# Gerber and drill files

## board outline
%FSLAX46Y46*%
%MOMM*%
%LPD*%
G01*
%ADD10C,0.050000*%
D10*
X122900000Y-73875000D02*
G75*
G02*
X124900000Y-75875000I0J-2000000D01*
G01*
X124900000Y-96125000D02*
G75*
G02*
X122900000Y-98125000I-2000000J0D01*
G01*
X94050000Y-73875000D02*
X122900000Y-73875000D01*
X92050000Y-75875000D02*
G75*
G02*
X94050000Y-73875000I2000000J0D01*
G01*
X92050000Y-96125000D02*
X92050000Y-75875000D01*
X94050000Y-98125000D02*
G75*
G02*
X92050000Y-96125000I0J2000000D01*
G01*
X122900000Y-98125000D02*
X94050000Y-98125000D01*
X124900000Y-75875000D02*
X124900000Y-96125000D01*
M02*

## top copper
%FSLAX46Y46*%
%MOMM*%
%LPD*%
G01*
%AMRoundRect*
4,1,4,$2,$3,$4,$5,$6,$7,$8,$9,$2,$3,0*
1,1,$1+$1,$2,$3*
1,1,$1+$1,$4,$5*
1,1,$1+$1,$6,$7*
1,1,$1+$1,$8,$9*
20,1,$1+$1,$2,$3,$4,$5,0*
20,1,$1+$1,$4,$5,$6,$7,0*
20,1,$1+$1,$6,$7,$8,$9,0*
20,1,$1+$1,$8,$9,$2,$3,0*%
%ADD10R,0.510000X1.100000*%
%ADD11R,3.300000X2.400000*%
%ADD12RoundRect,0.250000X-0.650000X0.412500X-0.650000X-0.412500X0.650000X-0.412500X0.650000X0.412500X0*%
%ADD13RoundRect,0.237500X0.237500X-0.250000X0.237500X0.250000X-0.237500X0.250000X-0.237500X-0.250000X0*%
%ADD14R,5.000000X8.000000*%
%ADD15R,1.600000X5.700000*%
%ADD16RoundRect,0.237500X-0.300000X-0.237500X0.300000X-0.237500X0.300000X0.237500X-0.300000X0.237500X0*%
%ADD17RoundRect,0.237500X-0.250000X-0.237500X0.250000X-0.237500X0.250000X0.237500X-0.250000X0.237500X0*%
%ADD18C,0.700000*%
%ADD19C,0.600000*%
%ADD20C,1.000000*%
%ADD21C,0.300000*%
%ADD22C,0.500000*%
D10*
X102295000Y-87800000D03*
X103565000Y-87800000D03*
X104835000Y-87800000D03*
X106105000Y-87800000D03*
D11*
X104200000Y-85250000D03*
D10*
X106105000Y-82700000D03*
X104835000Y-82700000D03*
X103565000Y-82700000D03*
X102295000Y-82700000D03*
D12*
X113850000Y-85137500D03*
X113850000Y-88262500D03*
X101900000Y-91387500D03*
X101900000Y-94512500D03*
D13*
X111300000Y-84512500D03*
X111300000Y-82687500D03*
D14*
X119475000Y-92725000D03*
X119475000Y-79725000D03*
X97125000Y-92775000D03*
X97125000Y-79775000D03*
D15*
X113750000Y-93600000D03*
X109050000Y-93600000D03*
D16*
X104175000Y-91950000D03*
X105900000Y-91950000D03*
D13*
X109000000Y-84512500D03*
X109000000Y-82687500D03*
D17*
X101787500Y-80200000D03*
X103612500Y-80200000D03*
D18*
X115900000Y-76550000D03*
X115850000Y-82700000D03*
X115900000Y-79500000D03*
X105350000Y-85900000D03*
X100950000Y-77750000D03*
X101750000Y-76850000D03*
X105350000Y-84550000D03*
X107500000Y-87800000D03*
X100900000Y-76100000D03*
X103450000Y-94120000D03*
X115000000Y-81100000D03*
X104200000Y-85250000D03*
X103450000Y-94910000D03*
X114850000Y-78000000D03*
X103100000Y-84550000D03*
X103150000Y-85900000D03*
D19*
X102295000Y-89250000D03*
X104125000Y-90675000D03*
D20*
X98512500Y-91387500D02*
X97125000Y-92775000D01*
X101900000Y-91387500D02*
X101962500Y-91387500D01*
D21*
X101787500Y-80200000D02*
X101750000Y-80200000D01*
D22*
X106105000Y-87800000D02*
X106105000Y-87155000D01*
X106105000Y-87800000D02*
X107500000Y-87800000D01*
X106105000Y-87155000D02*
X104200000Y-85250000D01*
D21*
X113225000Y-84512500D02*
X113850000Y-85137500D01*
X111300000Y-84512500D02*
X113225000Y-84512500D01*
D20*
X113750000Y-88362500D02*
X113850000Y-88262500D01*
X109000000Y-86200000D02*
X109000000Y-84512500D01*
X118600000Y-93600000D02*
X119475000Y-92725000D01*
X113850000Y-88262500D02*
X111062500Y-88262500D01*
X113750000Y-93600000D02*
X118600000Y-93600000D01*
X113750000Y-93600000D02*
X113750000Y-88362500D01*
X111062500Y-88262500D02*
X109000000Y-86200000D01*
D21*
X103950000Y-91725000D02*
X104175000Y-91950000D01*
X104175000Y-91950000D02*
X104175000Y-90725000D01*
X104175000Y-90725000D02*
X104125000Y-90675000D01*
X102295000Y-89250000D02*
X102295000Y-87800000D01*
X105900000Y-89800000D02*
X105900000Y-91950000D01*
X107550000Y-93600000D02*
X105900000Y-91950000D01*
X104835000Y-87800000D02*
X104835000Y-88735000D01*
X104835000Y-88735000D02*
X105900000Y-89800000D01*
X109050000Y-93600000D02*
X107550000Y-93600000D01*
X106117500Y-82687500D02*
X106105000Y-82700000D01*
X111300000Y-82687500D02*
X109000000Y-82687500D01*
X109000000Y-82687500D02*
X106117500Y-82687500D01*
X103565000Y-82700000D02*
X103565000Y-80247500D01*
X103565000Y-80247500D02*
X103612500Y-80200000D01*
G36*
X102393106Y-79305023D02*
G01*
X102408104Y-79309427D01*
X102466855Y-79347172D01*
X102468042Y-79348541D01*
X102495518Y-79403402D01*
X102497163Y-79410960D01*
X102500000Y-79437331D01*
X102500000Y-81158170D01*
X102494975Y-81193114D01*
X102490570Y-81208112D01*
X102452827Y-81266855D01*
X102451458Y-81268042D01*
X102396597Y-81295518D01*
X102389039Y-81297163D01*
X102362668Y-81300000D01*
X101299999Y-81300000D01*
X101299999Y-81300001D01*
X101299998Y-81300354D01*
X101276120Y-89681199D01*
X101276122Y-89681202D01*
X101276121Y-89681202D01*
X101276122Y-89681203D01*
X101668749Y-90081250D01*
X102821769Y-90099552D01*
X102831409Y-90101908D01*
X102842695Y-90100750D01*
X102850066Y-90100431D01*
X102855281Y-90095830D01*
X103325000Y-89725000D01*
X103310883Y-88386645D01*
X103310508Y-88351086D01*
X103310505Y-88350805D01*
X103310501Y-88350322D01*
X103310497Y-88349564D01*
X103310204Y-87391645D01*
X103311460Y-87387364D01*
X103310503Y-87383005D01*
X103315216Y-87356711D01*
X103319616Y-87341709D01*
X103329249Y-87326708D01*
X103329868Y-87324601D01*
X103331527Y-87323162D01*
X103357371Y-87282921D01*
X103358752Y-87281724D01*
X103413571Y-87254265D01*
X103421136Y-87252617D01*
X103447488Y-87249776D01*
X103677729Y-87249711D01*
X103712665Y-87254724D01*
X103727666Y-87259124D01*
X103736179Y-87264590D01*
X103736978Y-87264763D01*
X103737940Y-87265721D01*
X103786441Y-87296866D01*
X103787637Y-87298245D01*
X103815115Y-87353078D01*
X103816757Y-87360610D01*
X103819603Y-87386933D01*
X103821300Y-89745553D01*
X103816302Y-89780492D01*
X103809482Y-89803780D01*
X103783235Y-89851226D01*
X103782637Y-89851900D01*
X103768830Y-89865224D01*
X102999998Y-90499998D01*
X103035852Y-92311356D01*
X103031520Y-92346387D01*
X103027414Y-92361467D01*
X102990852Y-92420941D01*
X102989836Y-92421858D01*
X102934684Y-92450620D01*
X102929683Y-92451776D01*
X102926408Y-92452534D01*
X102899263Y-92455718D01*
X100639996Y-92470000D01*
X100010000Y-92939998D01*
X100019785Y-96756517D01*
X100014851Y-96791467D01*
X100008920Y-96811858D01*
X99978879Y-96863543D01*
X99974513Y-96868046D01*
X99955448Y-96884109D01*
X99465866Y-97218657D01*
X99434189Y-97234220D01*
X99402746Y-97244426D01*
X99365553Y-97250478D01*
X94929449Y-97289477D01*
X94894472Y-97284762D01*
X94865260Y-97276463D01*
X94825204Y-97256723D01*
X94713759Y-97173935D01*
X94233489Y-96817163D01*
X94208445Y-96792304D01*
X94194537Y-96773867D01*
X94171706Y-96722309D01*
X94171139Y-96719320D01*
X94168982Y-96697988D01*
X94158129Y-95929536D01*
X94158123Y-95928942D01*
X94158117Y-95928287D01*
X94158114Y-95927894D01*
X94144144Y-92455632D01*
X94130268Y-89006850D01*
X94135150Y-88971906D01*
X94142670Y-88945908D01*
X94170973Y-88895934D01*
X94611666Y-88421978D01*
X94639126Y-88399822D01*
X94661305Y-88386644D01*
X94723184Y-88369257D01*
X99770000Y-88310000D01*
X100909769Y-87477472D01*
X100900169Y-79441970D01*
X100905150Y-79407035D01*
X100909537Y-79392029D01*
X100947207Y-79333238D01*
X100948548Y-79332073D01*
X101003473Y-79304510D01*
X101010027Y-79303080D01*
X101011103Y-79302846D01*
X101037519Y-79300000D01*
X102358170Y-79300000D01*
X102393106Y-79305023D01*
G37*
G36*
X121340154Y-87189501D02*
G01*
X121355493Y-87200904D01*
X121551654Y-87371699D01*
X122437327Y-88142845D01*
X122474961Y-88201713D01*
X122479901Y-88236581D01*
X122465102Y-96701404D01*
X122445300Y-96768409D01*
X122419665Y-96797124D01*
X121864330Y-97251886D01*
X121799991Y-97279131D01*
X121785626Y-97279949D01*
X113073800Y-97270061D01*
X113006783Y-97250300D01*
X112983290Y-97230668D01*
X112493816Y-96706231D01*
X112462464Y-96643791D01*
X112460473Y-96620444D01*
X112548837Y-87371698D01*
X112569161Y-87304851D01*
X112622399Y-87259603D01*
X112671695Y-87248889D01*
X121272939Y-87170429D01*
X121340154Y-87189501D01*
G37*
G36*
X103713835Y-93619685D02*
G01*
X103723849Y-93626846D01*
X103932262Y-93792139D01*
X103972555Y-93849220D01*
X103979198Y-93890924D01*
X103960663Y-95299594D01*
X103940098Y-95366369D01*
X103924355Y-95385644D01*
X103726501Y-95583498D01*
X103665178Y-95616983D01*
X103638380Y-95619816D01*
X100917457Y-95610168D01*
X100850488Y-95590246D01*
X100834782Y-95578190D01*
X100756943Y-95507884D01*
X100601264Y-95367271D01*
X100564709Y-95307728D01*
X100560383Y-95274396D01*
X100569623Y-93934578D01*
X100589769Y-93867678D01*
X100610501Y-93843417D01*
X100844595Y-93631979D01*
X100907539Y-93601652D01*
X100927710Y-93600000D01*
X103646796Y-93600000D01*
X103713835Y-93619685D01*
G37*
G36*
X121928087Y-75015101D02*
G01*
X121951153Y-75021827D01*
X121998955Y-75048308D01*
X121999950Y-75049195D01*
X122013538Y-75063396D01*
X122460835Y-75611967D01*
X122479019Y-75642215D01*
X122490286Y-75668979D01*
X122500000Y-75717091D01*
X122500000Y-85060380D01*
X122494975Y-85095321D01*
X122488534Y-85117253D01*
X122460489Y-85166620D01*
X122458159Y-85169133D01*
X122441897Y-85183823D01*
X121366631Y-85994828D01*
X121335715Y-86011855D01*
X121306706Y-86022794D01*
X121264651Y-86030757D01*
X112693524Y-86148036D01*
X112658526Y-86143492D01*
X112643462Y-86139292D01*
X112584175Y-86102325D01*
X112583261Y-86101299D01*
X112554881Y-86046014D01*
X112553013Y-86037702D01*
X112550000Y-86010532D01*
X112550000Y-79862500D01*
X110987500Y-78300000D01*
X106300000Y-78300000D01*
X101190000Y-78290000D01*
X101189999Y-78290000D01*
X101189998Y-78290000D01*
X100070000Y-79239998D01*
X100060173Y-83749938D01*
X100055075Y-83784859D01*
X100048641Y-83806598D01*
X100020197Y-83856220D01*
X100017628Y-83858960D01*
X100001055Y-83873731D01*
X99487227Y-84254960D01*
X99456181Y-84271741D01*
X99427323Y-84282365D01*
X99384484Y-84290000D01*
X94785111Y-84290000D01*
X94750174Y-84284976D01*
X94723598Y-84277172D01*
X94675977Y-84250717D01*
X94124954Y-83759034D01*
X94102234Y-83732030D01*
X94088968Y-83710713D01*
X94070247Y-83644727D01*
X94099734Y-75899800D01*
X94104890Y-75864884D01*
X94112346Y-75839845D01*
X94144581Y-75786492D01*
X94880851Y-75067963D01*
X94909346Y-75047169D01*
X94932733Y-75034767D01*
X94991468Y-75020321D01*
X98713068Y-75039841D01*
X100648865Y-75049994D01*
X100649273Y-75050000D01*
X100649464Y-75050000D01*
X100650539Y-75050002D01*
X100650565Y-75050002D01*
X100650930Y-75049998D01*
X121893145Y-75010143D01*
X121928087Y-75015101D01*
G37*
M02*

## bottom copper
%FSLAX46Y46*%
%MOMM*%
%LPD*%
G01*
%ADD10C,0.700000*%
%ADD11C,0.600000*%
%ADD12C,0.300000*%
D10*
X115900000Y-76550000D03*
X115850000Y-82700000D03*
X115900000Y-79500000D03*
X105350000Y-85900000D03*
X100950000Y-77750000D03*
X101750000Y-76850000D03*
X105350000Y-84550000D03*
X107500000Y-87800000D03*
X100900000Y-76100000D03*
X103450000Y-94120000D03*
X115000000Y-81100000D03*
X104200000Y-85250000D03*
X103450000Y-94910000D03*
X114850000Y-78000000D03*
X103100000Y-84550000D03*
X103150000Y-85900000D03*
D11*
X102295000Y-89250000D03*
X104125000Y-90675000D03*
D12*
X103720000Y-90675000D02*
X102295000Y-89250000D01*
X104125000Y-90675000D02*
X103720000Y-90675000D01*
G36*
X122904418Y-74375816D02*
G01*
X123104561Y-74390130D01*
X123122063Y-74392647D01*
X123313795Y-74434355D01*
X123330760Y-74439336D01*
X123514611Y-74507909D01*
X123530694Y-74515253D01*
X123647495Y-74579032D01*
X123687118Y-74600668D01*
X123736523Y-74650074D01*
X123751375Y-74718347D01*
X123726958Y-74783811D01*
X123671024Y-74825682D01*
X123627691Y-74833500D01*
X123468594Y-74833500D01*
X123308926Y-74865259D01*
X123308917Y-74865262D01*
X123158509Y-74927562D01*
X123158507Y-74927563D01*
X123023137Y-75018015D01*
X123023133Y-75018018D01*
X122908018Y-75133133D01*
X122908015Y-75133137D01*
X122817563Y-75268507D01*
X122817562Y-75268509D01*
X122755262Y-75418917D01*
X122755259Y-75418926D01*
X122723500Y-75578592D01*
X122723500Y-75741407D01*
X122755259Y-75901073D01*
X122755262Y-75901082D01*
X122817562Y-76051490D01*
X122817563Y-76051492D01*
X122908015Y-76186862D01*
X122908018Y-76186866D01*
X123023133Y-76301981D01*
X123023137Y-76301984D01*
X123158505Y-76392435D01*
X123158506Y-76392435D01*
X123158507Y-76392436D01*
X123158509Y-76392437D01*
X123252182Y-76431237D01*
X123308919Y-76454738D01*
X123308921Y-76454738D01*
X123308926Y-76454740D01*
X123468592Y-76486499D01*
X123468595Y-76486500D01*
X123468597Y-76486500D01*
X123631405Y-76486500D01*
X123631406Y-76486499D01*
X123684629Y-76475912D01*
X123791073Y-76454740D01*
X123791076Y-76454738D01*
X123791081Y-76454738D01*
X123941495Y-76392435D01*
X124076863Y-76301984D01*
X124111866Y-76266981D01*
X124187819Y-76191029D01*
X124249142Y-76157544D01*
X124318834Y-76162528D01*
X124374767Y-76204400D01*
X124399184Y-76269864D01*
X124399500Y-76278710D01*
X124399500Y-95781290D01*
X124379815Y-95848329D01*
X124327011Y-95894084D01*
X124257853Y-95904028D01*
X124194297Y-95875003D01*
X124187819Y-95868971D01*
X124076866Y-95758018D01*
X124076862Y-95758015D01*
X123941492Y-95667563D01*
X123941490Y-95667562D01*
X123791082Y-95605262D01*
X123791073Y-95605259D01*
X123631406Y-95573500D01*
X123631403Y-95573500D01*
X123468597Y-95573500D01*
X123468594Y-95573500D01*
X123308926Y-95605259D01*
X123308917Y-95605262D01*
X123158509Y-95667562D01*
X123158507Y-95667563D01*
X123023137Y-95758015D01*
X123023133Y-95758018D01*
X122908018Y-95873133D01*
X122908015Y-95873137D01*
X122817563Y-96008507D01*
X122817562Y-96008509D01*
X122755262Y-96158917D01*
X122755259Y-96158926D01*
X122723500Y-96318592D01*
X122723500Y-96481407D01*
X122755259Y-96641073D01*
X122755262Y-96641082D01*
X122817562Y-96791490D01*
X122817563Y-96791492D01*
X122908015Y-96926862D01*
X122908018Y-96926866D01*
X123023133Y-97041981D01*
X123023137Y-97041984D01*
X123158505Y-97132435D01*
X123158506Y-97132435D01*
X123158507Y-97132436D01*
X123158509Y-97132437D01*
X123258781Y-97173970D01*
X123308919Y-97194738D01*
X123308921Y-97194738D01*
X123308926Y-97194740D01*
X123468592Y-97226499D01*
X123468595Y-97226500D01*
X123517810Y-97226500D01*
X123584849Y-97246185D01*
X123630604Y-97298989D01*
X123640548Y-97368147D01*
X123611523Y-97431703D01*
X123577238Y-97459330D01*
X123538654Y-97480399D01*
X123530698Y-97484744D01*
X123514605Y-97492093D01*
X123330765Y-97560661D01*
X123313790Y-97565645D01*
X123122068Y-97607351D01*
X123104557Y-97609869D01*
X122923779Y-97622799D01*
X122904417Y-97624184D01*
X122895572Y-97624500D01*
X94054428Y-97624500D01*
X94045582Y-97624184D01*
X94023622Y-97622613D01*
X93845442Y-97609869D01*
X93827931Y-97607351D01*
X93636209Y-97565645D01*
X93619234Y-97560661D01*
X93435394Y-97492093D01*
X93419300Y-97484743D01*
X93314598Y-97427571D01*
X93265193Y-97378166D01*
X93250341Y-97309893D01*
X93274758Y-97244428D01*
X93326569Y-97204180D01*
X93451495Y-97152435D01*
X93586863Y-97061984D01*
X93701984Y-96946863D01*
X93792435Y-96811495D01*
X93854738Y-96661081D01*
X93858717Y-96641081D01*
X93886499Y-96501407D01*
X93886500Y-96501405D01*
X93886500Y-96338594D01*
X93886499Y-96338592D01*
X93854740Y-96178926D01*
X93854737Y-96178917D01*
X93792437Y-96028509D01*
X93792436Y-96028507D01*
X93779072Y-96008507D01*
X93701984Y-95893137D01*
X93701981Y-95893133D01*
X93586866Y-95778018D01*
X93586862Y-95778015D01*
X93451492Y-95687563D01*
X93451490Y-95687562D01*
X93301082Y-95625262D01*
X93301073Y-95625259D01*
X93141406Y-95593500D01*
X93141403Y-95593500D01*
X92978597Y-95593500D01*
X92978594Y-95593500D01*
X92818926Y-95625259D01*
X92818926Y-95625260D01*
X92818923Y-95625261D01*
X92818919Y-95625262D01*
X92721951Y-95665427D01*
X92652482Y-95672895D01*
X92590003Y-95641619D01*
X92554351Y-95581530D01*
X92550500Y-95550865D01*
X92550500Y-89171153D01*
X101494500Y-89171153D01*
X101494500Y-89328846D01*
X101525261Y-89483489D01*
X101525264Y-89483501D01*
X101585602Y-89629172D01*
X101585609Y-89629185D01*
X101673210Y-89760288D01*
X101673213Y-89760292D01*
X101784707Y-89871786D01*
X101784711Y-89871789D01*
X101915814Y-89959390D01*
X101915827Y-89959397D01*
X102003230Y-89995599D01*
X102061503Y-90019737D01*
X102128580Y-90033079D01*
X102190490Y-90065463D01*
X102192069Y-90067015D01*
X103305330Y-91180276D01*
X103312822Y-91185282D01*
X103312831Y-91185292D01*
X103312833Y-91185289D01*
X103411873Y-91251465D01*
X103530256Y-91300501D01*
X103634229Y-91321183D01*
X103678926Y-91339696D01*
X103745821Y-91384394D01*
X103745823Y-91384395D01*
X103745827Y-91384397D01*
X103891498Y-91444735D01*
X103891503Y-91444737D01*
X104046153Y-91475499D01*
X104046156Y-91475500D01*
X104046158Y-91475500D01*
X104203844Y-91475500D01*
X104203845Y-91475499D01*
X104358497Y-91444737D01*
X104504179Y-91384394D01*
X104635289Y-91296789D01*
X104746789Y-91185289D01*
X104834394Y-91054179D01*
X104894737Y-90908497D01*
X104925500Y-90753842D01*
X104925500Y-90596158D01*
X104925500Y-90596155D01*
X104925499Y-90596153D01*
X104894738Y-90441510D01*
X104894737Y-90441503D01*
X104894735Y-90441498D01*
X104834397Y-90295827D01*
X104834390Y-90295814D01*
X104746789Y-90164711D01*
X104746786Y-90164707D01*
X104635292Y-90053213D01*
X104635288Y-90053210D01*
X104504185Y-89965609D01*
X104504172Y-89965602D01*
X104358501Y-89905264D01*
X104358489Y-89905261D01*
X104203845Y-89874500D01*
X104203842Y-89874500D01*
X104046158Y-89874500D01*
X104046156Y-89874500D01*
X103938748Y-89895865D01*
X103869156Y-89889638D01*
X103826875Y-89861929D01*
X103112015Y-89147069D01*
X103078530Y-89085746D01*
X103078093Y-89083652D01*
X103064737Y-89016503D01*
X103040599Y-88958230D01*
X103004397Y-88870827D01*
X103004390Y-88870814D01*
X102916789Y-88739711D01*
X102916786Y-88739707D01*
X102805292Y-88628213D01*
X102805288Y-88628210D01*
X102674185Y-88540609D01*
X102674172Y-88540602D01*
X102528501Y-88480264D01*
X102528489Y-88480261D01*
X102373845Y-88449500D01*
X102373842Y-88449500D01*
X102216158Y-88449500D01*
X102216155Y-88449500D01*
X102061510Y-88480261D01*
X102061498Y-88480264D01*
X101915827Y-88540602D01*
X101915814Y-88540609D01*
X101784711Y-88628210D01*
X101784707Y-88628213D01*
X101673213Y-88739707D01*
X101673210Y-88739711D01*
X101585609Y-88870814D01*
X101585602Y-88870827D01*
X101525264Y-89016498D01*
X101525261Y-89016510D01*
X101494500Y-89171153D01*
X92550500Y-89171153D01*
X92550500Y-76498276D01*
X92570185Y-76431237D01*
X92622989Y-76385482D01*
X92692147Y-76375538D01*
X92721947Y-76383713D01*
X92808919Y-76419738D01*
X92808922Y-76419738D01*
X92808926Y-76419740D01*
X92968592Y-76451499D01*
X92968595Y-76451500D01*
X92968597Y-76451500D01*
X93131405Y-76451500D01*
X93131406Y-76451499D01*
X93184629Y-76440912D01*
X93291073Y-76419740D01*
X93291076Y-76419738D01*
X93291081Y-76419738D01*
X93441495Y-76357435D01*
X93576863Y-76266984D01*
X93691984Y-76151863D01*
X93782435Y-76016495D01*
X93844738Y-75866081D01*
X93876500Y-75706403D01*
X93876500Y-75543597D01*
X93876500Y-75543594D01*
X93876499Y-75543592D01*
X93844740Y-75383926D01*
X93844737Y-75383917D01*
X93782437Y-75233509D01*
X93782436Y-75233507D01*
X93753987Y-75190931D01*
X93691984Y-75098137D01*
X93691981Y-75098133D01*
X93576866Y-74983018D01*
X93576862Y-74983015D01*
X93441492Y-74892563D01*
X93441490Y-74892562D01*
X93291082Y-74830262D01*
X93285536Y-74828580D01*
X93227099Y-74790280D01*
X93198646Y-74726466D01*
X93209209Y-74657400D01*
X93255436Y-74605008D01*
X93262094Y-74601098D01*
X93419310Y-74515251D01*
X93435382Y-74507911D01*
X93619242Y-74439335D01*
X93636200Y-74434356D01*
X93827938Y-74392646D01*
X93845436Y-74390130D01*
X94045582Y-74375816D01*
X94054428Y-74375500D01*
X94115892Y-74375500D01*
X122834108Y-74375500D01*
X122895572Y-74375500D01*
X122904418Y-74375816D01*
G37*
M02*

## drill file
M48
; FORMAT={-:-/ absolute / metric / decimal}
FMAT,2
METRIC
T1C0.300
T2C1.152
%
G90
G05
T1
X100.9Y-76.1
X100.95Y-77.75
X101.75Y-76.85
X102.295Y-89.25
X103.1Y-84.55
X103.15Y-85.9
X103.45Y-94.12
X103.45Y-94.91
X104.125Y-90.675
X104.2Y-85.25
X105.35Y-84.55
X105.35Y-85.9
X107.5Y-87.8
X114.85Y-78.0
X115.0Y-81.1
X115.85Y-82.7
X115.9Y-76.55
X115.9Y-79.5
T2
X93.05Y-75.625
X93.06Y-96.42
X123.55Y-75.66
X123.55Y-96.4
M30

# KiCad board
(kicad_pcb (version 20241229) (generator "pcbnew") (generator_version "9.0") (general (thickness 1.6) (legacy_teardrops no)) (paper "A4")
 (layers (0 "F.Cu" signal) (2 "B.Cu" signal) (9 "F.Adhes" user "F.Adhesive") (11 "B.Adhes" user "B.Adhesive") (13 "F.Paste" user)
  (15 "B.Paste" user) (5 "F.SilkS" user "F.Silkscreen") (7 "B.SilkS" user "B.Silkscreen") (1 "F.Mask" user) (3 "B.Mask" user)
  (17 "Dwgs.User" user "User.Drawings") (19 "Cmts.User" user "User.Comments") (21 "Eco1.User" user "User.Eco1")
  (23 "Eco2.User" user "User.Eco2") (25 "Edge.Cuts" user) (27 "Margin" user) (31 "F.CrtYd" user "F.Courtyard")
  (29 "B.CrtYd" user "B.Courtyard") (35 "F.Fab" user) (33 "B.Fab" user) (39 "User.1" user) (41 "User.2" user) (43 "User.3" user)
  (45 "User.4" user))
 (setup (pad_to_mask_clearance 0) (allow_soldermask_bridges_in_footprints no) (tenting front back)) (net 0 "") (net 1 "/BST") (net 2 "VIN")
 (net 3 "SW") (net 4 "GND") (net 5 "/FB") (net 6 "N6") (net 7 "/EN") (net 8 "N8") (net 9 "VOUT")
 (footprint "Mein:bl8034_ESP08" (layer "F.Cu") (at 104.2 85.25 90)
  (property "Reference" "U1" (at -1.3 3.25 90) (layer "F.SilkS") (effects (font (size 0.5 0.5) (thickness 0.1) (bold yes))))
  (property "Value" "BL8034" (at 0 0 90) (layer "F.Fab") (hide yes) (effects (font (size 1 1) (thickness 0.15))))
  (pad "1" smd rect (at -2.55 -1.905) (size 0.51 1.1) (layers "F.Cu" "F.Mask" "F.Paste") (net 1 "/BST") (thermal_bridge_angle 45))
  (pad "2" smd rect (at -2.55 -0.635) (size 0.51 1.1) (layers "F.Cu" "F.Mask" "F.Paste") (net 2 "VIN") (thermal_bridge_angle 45))
  (pad "3" smd rect (at -2.55 0.635) (size 0.51 1.1) (layers "F.Cu" "F.Mask" "F.Paste") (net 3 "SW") (thermal_bridge_angle 45))
  (pad "4" smd rect (at -2.55 1.905) (size 0.51 1.1) (layers "F.Cu" "F.Mask" "F.Paste") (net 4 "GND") (thermal_bridge_angle 45))
  (pad "4" smd rect (at 0 0) (size 3.3 2.4) (layers "F.Cu" "F.Mask" "F.Paste") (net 4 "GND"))
  (pad "5" smd rect (at 2.55 1.905) (size 0.51 1.1) (layers "F.Cu" "F.Mask" "F.Paste") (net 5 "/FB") (thermal_bridge_angle 45))
  (pad "6" smd rect (at 2.55 0.635) (size 0.51 1.1) (layers "F.Cu" "F.Mask" "F.Paste") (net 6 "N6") (thermal_bridge_angle 45))
  (pad "7" smd rect (at 2.55 -0.635) (size 0.51 1.1) (layers "F.Cu" "F.Mask" "F.Paste") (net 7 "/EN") (thermal_bridge_angle 45))
  (pad "8" smd rect (at 2.55 -1.905) (size 0.51 1.1) (layers "F.Cu" "F.Mask" "F.Paste") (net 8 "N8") (thermal_bridge_angle 45)))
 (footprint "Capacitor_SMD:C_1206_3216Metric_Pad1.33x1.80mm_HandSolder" (layer "F.Cu") (at 113.85 86.7 -90)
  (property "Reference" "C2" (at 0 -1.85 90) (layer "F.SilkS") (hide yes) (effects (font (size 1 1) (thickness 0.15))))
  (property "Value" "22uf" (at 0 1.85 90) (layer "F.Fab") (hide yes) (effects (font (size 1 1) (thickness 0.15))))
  (pad "1" smd roundrect (at -1.5625 0 270) (size 1.325 1.8) (layers "F.Cu" "F.Mask" "F.Paste") (roundrect_rratio 0.188679) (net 4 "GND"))
  (pad "2" smd roundrect (at 1.5625 0 270) (size 1.325 1.8) (layers "F.Cu" "F.Mask" "F.Paste") (roundrect_rratio 0.188679) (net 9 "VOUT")))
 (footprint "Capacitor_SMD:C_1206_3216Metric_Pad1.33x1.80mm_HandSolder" (layer "F.Cu") (at 101.9 92.95 -90)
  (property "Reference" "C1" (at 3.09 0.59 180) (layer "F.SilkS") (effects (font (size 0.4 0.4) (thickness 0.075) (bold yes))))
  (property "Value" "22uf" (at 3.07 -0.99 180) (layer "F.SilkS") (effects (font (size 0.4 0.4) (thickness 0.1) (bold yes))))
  (pad "1" smd roundrect (at -1.5625 0 270) (size 1.325 1.8) (layers "F.Cu" "F.Mask" "F.Paste") (roundrect_rratio 0.188679) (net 2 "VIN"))
  (pad "2" smd roundrect (at 1.5625 0 270) (size 1.325 1.8) (layers "F.Cu" "F.Mask" "F.Paste") (roundrect_rratio 0.188679) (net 4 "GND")))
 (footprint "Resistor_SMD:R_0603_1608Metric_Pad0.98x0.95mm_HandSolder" (layer "F.Cu") (at 111.3 83.6 90)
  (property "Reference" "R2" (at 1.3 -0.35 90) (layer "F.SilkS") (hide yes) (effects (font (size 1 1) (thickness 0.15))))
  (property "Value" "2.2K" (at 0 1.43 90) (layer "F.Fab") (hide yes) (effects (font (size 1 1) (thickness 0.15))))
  (pad "1" smd roundrect (at -0.9125 0 90) (size 0.975 0.95) (layers "F.Cu" "F.Mask" "F.Paste") (roundrect_rratio 0.25) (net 4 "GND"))
  (pad "2" smd roundrect (at 0.9125 0 90) (size 0.975 0.95) (layers "F.Cu" "F.Mask" "F.Paste") (roundrect_rratio 0.25) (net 5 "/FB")))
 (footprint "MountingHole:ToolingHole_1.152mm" (layer "F.Cu") (at 123.55 75.66)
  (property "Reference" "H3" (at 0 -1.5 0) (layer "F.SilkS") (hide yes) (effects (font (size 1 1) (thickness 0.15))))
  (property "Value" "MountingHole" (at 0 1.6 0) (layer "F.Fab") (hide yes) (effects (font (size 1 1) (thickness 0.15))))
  (pad "" np_thru_hole circle (at 0 0) (size 1.152 1.152) (drill 1.152) (layers "*.Cu" "*.Mask") (solder_mask_margin 0.074))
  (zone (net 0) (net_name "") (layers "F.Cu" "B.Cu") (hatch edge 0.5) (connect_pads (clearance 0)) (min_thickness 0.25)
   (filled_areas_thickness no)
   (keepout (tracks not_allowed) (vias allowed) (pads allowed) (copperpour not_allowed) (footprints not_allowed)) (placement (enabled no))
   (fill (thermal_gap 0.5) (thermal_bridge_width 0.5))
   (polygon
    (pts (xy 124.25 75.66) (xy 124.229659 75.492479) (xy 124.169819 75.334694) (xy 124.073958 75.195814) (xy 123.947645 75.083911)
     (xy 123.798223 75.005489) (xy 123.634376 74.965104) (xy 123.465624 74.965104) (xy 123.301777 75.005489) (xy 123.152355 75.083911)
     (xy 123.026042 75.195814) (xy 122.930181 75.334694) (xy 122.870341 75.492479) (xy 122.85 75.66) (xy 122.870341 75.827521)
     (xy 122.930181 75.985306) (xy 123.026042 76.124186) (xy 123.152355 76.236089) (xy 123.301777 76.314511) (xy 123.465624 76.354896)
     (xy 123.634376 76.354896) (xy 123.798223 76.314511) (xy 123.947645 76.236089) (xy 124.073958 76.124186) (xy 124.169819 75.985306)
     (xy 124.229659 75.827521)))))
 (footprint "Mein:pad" (layer "F.Cu") (at 116.975 102.225 180)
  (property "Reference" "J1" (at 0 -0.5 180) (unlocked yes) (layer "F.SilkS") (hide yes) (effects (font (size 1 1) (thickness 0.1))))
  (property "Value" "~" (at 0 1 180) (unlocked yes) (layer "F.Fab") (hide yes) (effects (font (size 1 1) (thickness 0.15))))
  (pad "1" smd rect (at -2.5 9.5 270) (size 8 5) (layers "F.Cu" "F.Mask" "F.Paste") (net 9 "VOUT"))
  (pad "2" smd rect (at -2.5 22.5 270) (size 8 5) (layers "F.Cu" "F.Mask" "F.Paste") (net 4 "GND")))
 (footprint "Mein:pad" (layer "F.Cu") (at 94.625 102.275 180)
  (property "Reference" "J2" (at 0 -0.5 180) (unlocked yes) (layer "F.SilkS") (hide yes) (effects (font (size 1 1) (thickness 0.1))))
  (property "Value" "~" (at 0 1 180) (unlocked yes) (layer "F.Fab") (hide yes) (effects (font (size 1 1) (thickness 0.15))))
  (pad "1" smd rect (at -2.5 9.5 270) (size 8 5) (layers "F.Cu" "F.Mask" "F.Paste") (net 2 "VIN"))
  (pad "2" smd rect (at -2.5 22.5 270) (size 8 5) (layers "F.Cu" "F.Mask" "F.Paste") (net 4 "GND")))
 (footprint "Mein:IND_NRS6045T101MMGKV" (layer "F.Cu") (at 111.4 93.6 180)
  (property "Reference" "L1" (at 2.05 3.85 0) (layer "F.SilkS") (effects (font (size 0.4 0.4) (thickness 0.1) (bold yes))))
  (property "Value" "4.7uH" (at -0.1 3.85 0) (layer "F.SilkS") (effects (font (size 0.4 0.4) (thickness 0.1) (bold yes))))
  (pad "1" smd rect (at -2.35 0 180) (size 1.6 5.7) (layers "F.Cu" "F.Mask" "F.Paste") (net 9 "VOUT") (solder_mask_margin 0.102))
  (pad "2" smd rect (at 2.35 0 180) (size 1.6 5.7) (layers "F.Cu" "F.Mask" "F.Paste") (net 3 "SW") (solder_mask_margin 0.102)))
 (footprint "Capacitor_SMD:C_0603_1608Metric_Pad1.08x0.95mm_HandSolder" (layer "F.Cu") (at 105.0375 91.95)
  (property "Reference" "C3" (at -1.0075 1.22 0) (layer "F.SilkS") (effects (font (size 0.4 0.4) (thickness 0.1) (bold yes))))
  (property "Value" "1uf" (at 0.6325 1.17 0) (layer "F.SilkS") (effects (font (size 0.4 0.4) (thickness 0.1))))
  (pad "1" smd roundrect (at -0.8625 0) (size 1.075 0.95) (layers "F.Cu" "F.Mask" "F.Paste") (roundrect_rratio 0.25) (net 1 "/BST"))
  (pad "2" smd roundrect (at 0.8625 0) (size 1.075 0.95) (layers "F.Cu" "F.Mask" "F.Paste") (roundrect_rratio 0.25) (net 3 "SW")))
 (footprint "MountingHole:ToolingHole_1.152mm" (layer "F.Cu") (at 93.05 75.625)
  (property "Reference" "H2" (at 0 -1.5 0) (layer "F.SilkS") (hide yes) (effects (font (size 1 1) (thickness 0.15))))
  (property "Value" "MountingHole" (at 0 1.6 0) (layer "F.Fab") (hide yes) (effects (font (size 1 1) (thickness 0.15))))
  (pad "" np_thru_hole circle (at 0 0) (size 1.152 1.152) (drill 1.152) (layers "*.Cu" "*.Mask") (solder_mask_margin 0.074))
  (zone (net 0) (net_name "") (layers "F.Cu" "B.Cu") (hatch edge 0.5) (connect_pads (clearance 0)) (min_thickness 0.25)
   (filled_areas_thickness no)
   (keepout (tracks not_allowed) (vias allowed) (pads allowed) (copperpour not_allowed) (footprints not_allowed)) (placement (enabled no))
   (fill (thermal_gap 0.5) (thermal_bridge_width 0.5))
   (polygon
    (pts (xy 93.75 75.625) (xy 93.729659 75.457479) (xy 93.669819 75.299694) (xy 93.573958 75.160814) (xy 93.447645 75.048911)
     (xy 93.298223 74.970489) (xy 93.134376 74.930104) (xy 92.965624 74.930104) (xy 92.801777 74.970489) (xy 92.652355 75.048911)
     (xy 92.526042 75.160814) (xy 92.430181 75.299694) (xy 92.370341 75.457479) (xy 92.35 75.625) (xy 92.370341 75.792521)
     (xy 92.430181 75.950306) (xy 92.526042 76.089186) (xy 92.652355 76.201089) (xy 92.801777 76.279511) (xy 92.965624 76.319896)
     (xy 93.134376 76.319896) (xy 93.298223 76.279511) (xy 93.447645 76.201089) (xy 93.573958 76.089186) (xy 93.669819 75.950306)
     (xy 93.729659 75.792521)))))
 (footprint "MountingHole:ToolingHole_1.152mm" (layer "F.Cu") (at 93.06 96.42)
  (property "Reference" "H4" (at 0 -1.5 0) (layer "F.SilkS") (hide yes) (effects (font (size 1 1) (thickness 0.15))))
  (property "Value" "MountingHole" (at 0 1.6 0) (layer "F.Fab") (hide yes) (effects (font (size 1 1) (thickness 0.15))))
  (pad "" np_thru_hole circle (at 0 0) (size 1.152 1.152) (drill 1.152) (layers "*.Cu" "*.Mask") (solder_mask_margin 0.074))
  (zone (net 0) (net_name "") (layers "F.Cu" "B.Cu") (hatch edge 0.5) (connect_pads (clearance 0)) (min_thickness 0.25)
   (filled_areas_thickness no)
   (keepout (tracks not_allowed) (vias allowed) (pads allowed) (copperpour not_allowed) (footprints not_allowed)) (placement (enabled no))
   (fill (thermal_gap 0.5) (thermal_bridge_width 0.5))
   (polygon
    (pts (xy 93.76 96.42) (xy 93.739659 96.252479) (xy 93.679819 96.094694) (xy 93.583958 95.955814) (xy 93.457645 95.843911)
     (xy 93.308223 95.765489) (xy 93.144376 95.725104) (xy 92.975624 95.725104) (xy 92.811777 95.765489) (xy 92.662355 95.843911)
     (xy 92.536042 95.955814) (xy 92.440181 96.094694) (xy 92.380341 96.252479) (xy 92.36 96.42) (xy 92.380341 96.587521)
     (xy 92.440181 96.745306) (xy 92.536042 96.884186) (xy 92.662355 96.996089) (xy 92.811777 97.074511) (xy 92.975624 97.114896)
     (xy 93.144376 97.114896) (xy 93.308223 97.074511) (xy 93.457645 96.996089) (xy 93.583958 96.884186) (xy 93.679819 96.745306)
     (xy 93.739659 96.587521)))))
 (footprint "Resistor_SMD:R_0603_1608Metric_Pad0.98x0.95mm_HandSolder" (layer "F.Cu") (at 109 83.6 90)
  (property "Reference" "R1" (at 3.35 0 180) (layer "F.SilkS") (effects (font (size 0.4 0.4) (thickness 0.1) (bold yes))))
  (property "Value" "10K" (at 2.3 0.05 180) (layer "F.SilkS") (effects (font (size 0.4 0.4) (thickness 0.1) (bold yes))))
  (pad "1" smd roundrect (at -0.9125 0 90) (size 0.975 0.95) (layers "F.Cu" "F.Mask" "F.Paste") (roundrect_rratio 0.25) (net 9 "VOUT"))
  (pad "2" smd roundrect (at 0.9125 0 90) (size 0.975 0.95) (layers "F.Cu" "F.Mask" "F.Paste") (roundrect_rratio 0.25) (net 5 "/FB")))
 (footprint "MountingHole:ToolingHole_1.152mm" (layer "F.Cu") (at 123.55 96.4)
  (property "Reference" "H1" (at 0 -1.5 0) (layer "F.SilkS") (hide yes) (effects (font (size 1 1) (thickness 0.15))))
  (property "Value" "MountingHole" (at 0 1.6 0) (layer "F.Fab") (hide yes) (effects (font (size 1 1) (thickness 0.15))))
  (pad "" np_thru_hole circle (at 0 0) (size 1.152 1.152) (drill 1.152) (layers "*.Cu" "*.Mask") (solder_mask_margin 0.074))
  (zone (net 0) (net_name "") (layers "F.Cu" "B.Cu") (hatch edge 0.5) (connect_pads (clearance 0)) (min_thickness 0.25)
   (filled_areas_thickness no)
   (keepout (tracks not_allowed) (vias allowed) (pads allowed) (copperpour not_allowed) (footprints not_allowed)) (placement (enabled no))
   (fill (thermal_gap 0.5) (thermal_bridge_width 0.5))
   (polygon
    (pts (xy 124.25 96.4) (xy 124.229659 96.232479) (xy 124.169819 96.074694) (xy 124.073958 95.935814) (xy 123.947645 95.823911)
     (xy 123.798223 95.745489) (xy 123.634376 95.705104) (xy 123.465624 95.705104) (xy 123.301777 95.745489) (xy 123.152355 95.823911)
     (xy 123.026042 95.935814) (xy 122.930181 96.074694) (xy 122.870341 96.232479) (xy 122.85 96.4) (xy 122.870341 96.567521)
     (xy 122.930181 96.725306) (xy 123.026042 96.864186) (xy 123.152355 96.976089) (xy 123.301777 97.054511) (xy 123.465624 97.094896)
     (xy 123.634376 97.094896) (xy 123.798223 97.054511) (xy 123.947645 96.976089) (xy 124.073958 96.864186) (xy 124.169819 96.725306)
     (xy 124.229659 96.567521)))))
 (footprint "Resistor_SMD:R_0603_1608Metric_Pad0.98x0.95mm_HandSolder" (layer "F.Cu") (at 102.7 80.2)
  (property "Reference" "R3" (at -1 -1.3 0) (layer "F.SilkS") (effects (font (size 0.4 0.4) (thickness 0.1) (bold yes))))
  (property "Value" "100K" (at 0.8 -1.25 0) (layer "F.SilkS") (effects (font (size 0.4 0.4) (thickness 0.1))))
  (pad "1" smd roundrect (at -0.9125 0) (size 0.975 0.95) (layers "F.Cu" "F.Mask" "F.Paste") (roundrect_rratio 0.25) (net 2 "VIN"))
  (pad "2" smd roundrect (at 0.9125 0) (size 0.975 0.95) (layers "F.Cu" "F.Mask" "F.Paste") (roundrect_rratio 0.25) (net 7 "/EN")))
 (gr_arc (start 122.9 73.875) (mid 124.314214 74.460786) (end 124.9 75.875) (stroke (width 0.05) (type default)) (layer "Edge.Cuts"))
 (gr_arc (start 124.9 96.125) (mid 124.314214 97.539214) (end 122.9 98.125) (stroke (width 0.05) (type default)) (layer "Edge.Cuts"))
 (gr_line (start 94.05 73.875) (end 122.9 73.875) (stroke (width 0.05) (type default)) (layer "Edge.Cuts"))
 (gr_arc (start 92.05 75.875) (mid 92.635786 74.460786) (end 94.05 73.875) (stroke (width 0.05) (type default)) (layer "Edge.Cuts"))
 (gr_line (start 92.05 96.125) (end 92.05 75.875) (stroke (width 0.05) (type default)) (layer "Edge.Cuts"))
 (gr_arc (start 94.05 98.125) (mid 92.635786 97.539214) (end 92.05 96.125) (stroke (width 0.05) (type default)) (layer "Edge.Cuts"))
 (gr_line (start 122.9 98.125) (end 94.05 98.125) (stroke (width 0.05) (type default)) (layer "Edge.Cuts"))
 (gr_line (start 124.9 75.875) (end 124.9 96.125) (stroke (width 0.05) (type default)) (layer "Edge.Cuts"))
 (segment (start 98.5125 91.3875) (end 97.125 92.775) (width 1) (layer "F.Cu") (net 2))
 (segment (start 101.9 91.3875) (end 101.9625 91.3875) (width 1) (layer "F.Cu") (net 2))
 (segment (start 101.7875 80.2) (end 101.75 80.2) (width 0.3) (layer "F.Cu") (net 2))
 (segment (start 106.105 87.8) (end 106.105 87.155) (width 0.5) (layer "F.Cu") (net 4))
 (segment (start 106.105 87.8) (end 107.5 87.8) (width 0.5) (layer "F.Cu") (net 4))
 (segment (start 106.105 87.155) (end 104.2 85.25) (width 0.5) (layer "F.Cu") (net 4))
 (segment (start 113.225 84.5125) (end 113.85 85.1375) (width 0.3) (layer "F.Cu") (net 4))
 (segment (start 111.3 84.5125) (end 113.225 84.5125) (width 0.3) (layer "F.Cu") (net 4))
 (via (at 115.9 76.55) (size 0.7) (drill 0.3) (layers "F.Cu" "B.Cu") (free yes) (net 4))
 (via (at 115.85 82.7) (size 0.7) (drill 0.3) (layers "F.Cu" "B.Cu") (free yes) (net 4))
 (via (at 115.9 79.5) (size 0.7) (drill 0.3) (layers "F.Cu" "B.Cu") (free yes) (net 4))
 (via (at 105.35 85.9) (size 0.7) (drill 0.3) (layers "F.Cu" "B.Cu") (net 4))
 (via (at 100.95 77.75) (size 0.7) (drill 0.3) (layers "F.Cu" "B.Cu") (free yes) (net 4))
 (via (at 101.75 76.85) (size 0.7) (drill 0.3) (layers "F.Cu" "B.Cu") (free yes) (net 4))
 (via (at 105.35 84.55) (size 0.7) (drill 0.3) (layers "F.Cu" "B.Cu") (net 4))
 (via (at 107.5 87.8) (size 0.7) (drill 0.3) (layers "F.Cu" "B.Cu") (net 4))
 (via (at 100.9 76.1) (size 0.7) (drill 0.3) (layers "F.Cu" "B.Cu") (free yes) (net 4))
 (via (at 103.45 94.12) (size 0.7) (drill 0.3) (layers "F.Cu" "B.Cu") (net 4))
 (via (at 115 81.1) (size 0.7) (drill 0.3) (layers "F.Cu" "B.Cu") (free yes) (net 4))
 (via (at 104.2 85.25) (size 0.7) (drill 0.3) (layers "F.Cu" "B.Cu") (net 4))
 (via (at 103.45 94.91) (size 0.7) (drill 0.3) (layers "F.Cu" "B.Cu") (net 4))
 (via (at 114.85 78) (size 0.7) (drill 0.3) (layers "F.Cu" "B.Cu") (free yes) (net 4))
 (via (at 103.1 84.55) (size 0.7) (drill 0.3) (layers "F.Cu" "B.Cu") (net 4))
 (via (at 103.15 85.9) (size 0.7) (drill 0.3) (layers "F.Cu" "B.Cu") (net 4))
 (segment (start 113.75 88.3625) (end 113.85 88.2625) (width 1) (layer "F.Cu") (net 9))
 (segment (start 109 86.2) (end 109 84.5125) (width 1) (layer "F.Cu") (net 9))
 (segment (start 118.6 93.6) (end 119.475 92.725) (width 1) (layer "F.Cu") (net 9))
 (segment (start 113.85 88.2625) (end 111.0625 88.2625) (width 1) (layer "F.Cu") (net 9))
 (segment (start 113.75 93.6) (end 118.6 93.6) (width 1) (layer "F.Cu") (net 9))
 (segment (start 113.75 93.6) (end 113.75 88.3625) (width 1) (layer "F.Cu") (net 9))
 (segment (start 111.0625 88.2625) (end 109 86.2) (width 1) (layer "F.Cu") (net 9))
 (segment (start 103.95 91.725) (end 104.175 91.95) (width 0.3) (layer "F.Cu") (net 1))
 (segment (start 104.175 91.95) (end 104.175 90.725) (width 0.3) (layer "F.Cu") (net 1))
 (segment (start 104.175 90.725) (end 104.125 90.675) (width 0.3) (layer "F.Cu") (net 1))
 (segment (start 102.295 89.25) (end 102.295 87.8) (width 0.3) (layer "F.Cu") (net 1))
 (via (at 102.295 89.25) (size 0.6) (drill 0.3) (layers "F.Cu" "B.Cu") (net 1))
 (via (at 104.125 90.675) (size 0.6) (drill 0.3) (layers "F.Cu" "B.Cu") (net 1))
 (segment (start 103.72 90.675) (end 102.295 89.25) (width 0.3) (layer "B.Cu") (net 1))
 (segment (start 104.125 90.675) (end 103.72 90.675) (width 0.3) (layer "B.Cu") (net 1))
 (segment (start 105.9 89.8) (end 105.9 91.95) (width 0.3) (layer "F.Cu") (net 3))
 (segment (start 107.55 93.6) (end 105.9 91.95) (width 0.3) (layer "F.Cu") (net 3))
 (segment (start 104.835 87.8) (end 104.835 88.735) (width 0.3) (layer "F.Cu") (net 3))
 (segment (start 104.835 88.735) (end 105.9 89.8) (width 0.3) (layer "F.Cu") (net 3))
 (segment (start 109.05 93.6) (end 107.55 93.6) (width 0.3) (layer "F.Cu") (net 3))
 (segment (start 106.1175 82.6875) (end 106.105 82.7) (width 0.3) (layer "F.Cu") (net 5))
 (segment (start 111.3 82.6875) (end 109 82.6875) (width 0.3) (layer "F.Cu") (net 5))
 (segment (start 109 82.6875) (end 106.1175 82.6875) (width 0.3) (layer "F.Cu") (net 5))
 (segment (start 103.565 82.7) (end 103.565 80.2475) (width 0.3) (layer "F.Cu") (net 7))
 (segment (start 103.565 80.2475) (end 103.6125 80.2) (width 0.3) (layer "F.Cu") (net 7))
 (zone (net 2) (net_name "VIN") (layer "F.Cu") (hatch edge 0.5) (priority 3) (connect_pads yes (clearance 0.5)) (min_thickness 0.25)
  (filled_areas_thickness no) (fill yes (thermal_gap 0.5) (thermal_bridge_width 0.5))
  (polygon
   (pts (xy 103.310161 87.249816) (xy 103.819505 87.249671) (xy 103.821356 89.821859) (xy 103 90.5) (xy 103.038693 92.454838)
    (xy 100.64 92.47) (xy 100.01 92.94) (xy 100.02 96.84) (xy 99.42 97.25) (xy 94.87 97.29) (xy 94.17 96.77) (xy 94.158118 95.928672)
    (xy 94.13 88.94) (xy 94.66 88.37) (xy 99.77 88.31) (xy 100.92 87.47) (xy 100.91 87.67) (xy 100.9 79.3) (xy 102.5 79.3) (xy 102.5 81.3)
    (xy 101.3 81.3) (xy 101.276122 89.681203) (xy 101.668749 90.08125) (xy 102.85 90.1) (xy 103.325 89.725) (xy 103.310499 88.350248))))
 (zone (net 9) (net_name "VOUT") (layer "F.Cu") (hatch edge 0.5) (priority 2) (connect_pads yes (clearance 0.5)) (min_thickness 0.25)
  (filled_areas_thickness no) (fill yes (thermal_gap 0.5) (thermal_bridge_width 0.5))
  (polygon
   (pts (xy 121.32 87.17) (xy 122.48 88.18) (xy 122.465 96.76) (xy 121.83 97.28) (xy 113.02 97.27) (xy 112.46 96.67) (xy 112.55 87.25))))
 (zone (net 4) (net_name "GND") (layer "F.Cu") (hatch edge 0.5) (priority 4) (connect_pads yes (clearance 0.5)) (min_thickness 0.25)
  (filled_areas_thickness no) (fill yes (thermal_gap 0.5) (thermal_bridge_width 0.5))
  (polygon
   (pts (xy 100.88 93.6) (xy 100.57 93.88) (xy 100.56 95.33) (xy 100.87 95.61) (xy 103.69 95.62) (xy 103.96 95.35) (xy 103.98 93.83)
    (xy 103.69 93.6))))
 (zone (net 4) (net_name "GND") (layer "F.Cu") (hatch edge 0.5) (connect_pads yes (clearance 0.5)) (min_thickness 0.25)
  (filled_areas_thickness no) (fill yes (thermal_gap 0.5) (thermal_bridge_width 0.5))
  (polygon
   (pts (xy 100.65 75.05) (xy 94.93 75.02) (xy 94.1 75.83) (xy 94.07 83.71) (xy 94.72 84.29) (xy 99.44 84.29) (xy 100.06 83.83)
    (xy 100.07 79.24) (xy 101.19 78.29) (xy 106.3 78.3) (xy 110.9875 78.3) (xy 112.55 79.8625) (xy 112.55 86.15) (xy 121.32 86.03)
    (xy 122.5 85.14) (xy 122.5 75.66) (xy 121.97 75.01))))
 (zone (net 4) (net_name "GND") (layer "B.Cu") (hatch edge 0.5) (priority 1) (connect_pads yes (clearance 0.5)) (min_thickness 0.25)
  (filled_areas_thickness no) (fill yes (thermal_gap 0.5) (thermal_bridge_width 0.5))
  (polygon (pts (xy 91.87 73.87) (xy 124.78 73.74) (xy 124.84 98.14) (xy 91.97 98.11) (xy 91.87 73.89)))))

